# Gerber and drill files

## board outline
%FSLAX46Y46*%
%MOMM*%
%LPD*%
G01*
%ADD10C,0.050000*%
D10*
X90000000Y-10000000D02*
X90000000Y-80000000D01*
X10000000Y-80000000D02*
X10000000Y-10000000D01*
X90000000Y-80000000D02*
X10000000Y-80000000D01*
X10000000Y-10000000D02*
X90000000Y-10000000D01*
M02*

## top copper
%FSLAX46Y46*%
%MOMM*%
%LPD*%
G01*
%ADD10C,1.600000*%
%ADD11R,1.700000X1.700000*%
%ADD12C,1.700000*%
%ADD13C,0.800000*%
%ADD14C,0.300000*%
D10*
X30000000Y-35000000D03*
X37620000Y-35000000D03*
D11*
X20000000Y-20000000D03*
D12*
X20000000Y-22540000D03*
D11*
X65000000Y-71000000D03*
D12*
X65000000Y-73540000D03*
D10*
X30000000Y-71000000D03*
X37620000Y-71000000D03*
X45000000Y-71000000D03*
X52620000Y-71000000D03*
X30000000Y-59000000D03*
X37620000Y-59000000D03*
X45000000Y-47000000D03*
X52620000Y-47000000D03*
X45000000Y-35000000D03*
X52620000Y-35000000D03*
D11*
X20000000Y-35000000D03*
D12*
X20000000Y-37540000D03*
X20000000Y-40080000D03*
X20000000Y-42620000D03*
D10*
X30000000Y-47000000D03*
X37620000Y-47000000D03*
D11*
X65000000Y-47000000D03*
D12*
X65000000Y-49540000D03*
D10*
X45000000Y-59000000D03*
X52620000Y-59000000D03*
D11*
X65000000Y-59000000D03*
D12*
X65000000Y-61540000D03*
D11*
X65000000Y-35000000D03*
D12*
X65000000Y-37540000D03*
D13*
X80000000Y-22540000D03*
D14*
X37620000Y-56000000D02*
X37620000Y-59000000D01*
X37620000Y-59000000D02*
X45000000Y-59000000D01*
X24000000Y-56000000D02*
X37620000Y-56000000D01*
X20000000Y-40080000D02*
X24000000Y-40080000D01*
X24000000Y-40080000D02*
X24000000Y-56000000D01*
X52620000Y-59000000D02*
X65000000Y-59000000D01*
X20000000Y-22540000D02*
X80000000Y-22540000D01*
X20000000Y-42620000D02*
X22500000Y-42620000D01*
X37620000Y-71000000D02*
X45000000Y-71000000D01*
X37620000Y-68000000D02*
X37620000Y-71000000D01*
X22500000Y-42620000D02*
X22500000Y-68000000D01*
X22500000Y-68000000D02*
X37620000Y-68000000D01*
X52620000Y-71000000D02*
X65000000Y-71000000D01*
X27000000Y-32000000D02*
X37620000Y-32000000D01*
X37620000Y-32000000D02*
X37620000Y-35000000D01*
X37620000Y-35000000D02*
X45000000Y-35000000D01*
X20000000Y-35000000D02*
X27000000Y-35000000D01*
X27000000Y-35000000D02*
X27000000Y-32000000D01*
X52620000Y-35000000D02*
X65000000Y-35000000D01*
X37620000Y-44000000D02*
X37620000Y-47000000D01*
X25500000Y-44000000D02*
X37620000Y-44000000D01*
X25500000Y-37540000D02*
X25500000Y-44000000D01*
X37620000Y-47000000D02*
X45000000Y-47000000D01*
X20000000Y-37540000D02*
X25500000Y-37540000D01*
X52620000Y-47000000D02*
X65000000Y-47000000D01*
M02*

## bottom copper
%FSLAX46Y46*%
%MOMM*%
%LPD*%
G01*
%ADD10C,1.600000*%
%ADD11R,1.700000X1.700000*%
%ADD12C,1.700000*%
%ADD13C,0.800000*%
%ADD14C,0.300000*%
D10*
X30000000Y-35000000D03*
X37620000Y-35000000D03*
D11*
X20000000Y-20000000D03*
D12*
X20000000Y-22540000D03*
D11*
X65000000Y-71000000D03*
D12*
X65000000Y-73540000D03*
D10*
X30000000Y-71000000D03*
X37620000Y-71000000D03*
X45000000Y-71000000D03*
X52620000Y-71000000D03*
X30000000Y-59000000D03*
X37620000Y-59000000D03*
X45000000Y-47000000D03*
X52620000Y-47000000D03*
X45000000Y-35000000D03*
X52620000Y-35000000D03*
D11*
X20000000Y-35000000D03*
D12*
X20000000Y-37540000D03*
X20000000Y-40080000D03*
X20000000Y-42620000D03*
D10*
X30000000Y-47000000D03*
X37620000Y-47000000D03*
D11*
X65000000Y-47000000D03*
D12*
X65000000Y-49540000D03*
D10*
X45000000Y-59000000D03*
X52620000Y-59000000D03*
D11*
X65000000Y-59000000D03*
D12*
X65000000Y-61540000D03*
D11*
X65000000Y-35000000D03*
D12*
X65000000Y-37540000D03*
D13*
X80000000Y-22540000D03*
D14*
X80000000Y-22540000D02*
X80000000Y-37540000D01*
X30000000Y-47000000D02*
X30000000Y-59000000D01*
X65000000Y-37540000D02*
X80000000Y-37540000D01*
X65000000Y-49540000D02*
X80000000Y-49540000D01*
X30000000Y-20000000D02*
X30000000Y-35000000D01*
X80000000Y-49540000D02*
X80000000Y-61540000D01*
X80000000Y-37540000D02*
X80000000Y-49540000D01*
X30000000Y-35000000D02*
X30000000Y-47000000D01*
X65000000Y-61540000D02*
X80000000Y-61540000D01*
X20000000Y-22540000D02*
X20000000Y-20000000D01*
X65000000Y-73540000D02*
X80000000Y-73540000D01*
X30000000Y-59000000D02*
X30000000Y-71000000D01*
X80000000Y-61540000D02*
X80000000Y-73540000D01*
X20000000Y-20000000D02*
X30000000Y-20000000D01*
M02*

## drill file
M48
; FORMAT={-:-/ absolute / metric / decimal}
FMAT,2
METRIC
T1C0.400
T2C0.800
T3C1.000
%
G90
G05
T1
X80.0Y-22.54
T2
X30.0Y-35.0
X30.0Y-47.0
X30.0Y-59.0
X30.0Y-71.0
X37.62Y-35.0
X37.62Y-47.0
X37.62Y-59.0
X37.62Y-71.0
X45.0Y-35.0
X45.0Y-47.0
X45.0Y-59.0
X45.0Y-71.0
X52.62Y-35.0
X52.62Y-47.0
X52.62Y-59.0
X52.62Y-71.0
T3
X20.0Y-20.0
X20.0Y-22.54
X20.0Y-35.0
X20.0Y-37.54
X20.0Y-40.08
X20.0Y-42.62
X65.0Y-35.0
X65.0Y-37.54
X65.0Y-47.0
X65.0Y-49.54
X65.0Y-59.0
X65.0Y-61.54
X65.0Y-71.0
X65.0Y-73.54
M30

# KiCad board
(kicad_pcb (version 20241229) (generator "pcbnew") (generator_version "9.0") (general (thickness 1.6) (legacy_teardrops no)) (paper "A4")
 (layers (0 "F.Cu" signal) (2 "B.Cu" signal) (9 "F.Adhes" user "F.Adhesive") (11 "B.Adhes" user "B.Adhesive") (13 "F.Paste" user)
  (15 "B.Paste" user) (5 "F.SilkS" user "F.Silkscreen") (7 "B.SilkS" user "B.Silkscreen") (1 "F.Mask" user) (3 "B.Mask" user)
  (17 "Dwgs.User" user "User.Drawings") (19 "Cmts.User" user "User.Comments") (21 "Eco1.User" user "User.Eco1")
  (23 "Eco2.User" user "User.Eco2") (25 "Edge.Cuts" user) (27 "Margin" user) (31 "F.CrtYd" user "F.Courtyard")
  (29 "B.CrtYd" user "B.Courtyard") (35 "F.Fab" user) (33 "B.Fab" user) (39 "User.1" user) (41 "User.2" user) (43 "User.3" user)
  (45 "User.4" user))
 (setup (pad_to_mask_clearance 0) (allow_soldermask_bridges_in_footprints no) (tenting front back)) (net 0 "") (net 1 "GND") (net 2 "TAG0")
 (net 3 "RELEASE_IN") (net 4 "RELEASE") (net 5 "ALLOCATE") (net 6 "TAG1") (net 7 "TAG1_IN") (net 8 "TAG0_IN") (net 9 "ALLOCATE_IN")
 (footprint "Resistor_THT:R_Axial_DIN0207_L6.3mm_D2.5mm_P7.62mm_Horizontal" (layer "F.Cu") (at 30 35)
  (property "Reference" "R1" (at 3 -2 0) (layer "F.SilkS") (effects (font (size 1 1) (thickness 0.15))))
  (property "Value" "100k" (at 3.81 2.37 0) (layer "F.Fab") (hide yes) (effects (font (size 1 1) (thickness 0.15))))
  (pad "1" thru_hole circle (at 0 0) (size 1.6 1.6) (drill 0.8) (layers "*.Cu" "*.Mask") (remove_unused_layers no) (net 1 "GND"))
  (pad "2" thru_hole circle (at 7.62 0) (size 1.6 1.6) (drill 0.8) (layers "*.Cu" "*.Mask") (remove_unused_layers no) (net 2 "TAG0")))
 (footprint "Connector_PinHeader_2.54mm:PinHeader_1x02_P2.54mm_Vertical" (layer "F.Cu") (at 20 20)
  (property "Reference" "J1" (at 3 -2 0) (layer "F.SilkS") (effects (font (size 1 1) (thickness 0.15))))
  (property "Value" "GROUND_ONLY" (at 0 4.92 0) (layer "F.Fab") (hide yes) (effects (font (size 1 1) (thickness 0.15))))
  (pad "1" thru_hole rect (at 0 0) (size 1.7 1.7) (drill 1) (layers "*.Cu" "*.Mask") (remove_unused_layers no) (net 1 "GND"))
  (pad "2" thru_hole circle (at 0 2.54) (size 1.7 1.7) (drill 1) (layers "*.Cu" "*.Mask") (remove_unused_layers no) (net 1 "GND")))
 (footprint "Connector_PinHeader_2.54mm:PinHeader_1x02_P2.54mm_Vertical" (layer "F.Cu") (at 65 71)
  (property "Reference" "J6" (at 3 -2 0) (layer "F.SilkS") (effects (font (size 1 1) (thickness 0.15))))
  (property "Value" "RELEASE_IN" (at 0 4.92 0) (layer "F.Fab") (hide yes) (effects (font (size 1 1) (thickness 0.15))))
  (pad "1" thru_hole rect (at 0 0) (size 1.7 1.7) (drill 1) (layers "*.Cu" "*.Mask") (remove_unused_layers no) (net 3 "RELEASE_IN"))
  (pad "2" thru_hole circle (at 0 2.54) (size 1.7 1.7) (drill 1) (layers "*.Cu" "*.Mask") (remove_unused_layers no) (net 1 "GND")))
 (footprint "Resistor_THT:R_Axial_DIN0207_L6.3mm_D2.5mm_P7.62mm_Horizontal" (layer "F.Cu") (at 30 71)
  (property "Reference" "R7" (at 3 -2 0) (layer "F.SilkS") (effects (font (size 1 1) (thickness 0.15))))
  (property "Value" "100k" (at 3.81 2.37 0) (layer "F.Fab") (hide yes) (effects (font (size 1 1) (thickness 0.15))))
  (pad "1" thru_hole circle (at 0 0) (size 1.6 1.6) (drill 0.8) (layers "*.Cu" "*.Mask") (remove_unused_layers no) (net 1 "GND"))
  (pad "2" thru_hole circle (at 7.62 0) (size 1.6 1.6) (drill 0.8) (layers "*.Cu" "*.Mask") (remove_unused_layers no) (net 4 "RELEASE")))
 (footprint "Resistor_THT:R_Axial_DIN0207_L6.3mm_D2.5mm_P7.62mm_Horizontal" (layer "F.Cu") (at 45 71)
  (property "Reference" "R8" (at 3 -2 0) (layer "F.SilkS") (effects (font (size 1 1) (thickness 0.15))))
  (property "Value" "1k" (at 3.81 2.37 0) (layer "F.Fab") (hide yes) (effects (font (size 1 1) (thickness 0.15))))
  (pad "1" thru_hole circle (at 0 0) (size 1.6 1.6) (drill 0.8) (layers "*.Cu" "*.Mask") (remove_unused_layers no) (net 4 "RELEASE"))
  (pad "2" thru_hole circle (at 7.62 0) (size 1.6 1.6) (drill 0.8) (layers "*.Cu" "*.Mask") (remove_unused_layers no) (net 3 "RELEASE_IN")))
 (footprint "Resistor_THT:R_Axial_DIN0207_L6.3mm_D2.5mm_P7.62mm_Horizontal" (layer "F.Cu") (at 30 59)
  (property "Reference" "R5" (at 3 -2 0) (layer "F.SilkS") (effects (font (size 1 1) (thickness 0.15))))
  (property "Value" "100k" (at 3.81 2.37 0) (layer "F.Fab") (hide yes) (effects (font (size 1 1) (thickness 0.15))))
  (pad "1" thru_hole circle (at 0 0) (size 1.6 1.6) (drill 0.8) (layers "*.Cu" "*.Mask") (remove_unused_layers no) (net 1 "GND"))
  (pad "2" thru_hole circle (at 7.62 0) (size 1.6 1.6) (drill 0.8) (layers "*.Cu" "*.Mask") (remove_unused_layers no) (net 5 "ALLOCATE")))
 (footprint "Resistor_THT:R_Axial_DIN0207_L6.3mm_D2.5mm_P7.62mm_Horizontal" (layer "F.Cu") (at 45 47)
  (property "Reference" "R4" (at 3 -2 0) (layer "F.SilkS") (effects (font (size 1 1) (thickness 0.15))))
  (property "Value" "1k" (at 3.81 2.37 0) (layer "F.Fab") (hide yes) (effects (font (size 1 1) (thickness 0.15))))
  (pad "1" thru_hole circle (at 0 0) (size 1.6 1.6) (drill 0.8) (layers "*.Cu" "*.Mask") (remove_unused_layers no) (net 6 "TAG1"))
  (pad "2" thru_hole circle (at 7.62 0) (size 1.6 1.6) (drill 0.8) (layers "*.Cu" "*.Mask") (remove_unused_layers no) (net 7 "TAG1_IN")))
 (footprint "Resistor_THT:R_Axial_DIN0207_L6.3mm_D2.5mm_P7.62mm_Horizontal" (layer "F.Cu") (at 45 35)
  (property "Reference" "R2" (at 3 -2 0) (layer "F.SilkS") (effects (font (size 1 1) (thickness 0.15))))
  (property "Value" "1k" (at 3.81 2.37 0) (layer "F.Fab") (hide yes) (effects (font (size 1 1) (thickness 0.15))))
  (pad "1" thru_hole circle (at 0 0) (size 1.6 1.6) (drill 0.8) (layers "*.Cu" "*.Mask") (remove_unused_layers no) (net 2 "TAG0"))
  (pad "2" thru_hole circle (at 7.62 0) (size 1.6 1.6) (drill 0.8) (layers "*.Cu" "*.Mask") (remove_unused_layers no) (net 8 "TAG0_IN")))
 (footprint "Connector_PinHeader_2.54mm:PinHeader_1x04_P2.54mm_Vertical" (layer "F.Cu") (at 20 35)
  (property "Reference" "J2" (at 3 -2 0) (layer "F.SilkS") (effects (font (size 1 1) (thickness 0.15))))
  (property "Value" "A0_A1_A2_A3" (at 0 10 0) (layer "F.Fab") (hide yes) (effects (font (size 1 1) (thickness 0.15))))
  (pad "1" thru_hole rect (at 0 0) (size 1.7 1.7) (drill 1) (layers "*.Cu" "*.Mask") (remove_unused_layers no) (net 2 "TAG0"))
  (pad "2" thru_hole circle (at 0 2.54) (size 1.7 1.7) (drill 1) (layers "*.Cu" "*.Mask") (remove_unused_layers no) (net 6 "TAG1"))
  (pad "3" thru_hole circle (at 0 5.08) (size 1.7 1.7) (drill 1) (layers "*.Cu" "*.Mask") (remove_unused_layers no) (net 5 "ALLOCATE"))
  (pad "4" thru_hole circle (at 0 7.62) (size 1.7 1.7) (drill 1) (layers "*.Cu" "*.Mask") (remove_unused_layers no) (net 4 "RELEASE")))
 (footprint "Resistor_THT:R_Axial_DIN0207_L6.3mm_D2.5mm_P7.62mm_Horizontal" (layer "F.Cu") (at 30 47)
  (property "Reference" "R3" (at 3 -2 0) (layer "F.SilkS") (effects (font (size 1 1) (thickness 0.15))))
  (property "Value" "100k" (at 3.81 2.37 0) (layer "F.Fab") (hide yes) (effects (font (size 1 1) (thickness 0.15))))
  (pad "1" thru_hole circle (at 0 0) (size 1.6 1.6) (drill 0.8) (layers "*.Cu" "*.Mask") (remove_unused_layers no) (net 1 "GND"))
  (pad "2" thru_hole circle (at 7.62 0) (size 1.6 1.6) (drill 0.8) (layers "*.Cu" "*.Mask") (remove_unused_layers no) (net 6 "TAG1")))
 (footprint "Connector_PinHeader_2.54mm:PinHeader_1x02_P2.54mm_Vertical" (layer "F.Cu") (at 65 47)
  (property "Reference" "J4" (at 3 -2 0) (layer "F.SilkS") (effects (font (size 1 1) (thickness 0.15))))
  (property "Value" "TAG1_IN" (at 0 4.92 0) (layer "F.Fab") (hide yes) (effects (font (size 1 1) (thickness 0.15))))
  (pad "1" thru_hole rect (at 0 0) (size 1.7 1.7) (drill 1) (layers "*.Cu" "*.Mask") (remove_unused_layers no) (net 7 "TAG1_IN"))
  (pad "2" thru_hole circle (at 0 2.54) (size 1.7 1.7) (drill 1) (layers "*.Cu" "*.Mask") (remove_unused_layers no) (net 1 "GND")))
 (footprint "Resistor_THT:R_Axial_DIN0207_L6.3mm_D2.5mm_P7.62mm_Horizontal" (layer "F.Cu") (at 45 59)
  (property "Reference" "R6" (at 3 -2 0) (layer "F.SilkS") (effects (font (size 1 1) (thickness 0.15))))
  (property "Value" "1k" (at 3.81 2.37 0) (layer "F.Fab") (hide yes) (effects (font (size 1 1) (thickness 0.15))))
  (pad "1" thru_hole circle (at 0 0) (size 1.6 1.6) (drill 0.8) (layers "*.Cu" "*.Mask") (remove_unused_layers no) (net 5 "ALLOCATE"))
  (pad "2" thru_hole circle (at 7.62 0) (size 1.6 1.6) (drill 0.8) (layers "*.Cu" "*.Mask") (remove_unused_layers no) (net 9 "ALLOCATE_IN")))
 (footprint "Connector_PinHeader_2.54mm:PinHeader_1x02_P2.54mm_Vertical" (layer "F.Cu") (at 65 59)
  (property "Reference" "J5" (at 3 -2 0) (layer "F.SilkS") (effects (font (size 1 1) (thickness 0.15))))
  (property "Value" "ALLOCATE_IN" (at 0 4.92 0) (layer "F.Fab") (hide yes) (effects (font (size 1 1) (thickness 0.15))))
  (pad "1" thru_hole rect (at 0 0) (size 1.7 1.7) (drill 1) (layers "*.Cu" "*.Mask") (remove_unused_layers no) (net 9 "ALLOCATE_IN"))
  (pad "2" thru_hole circle (at 0 2.54) (size 1.7 1.7) (drill 1) (layers "*.Cu" "*.Mask") (remove_unused_layers no) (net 1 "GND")))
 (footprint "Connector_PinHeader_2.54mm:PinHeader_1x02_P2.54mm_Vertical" (layer "F.Cu") (at 65 35)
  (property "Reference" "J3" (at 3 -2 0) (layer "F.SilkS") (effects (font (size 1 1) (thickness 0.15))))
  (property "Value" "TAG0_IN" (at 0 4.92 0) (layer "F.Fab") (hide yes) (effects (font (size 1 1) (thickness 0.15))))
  (pad "1" thru_hole rect (at 0 0) (size 1.7 1.7) (drill 1) (layers "*.Cu" "*.Mask") (remove_unused_layers no) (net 8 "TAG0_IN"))
  (pad "2" thru_hole circle (at 0 2.54) (size 1.7 1.7) (drill 1) (layers "*.Cu" "*.Mask") (remove_unused_layers no) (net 1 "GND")))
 (gr_line (start 90 10) (end 90 80) (stroke (width 0.05) (type default)) (layer "Edge.Cuts"))
 (gr_line (start 10 80) (end 10 10) (stroke (width 0.05) (type default)) (layer "Edge.Cuts"))
 (gr_line (start 90 80) (end 10 80) (stroke (width 0.05) (type default)) (layer "Edge.Cuts"))
 (gr_line (start 10 10) (end 90 10) (stroke (width 0.05) (type default)) (layer "Edge.Cuts"))
 (segment (start 37.62 56) (end 37.62 59) (width 0.3) (layer "F.Cu") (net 5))
 (segment (start 37.62 59) (end 45 59) (width 0.3) (layer "F.Cu") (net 5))
 (segment (start 24 56) (end 37.62 56) (width 0.3) (layer "F.Cu") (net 5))
 (segment (start 20 40.08) (end 24 40.08) (width 0.3) (layer "F.Cu") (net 5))
 (segment (start 24 40.08) (end 24 56) (width 0.3) (layer "F.Cu") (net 5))
 (segment (start 52.62 59) (end 65 59) (width 0.3) (layer "F.Cu") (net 9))
 (segment (start 20 22.54) (end 80 22.54) (width 0.3) (layer "F.Cu") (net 1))
 (via (at 80 22.54) (size 0.8) (drill 0.4) (layers "F.Cu" "B.Cu") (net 1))
 (segment (start 80 22.54) (end 80 37.54) (width 0.3) (layer "B.Cu") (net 1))
 (segment (start 30 47) (end 30 59) (width 0.3) (layer "B.Cu") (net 1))
 (segment (start 65 37.54) (end 80 37.54) (width 0.3) (layer "B.Cu") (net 1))
 (segment (start 65 49.54) (end 80 49.54) (width 0.3) (layer "B.Cu") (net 1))
 (segment (start 30 20) (end 30 35) (width 0.3) (layer "B.Cu") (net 1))
 (segment (start 80 49.54) (end 80 61.54) (width 0.3) (layer "B.Cu") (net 1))
 (segment (start 80 37.54) (end 80 49.54) (width 0.3) (layer "B.Cu") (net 1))
 (segment (start 30 35) (end 30 47) (width 0.3) (layer "B.Cu") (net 1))
 (segment (start 65 61.54) (end 80 61.54) (width 0.3) (layer "B.Cu") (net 1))
 (segment (start 20 22.54) (end 20 20) (width 0.3) (layer "B.Cu") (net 1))
 (segment (start 65 73.54) (end 80 73.54) (width 0.3) (layer "B.Cu") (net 1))
 (segment (start 30 59) (end 30 71) (width 0.3) (layer "B.Cu") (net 1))
 (segment (start 80 61.54) (end 80 73.54) (width 0.3) (layer "B.Cu") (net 1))
 (segment (start 20 20) (end 30 20) (width 0.3) (layer "B.Cu") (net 1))
 (segment (start 20 42.62) (end 22.5 42.62) (width 0.3) (layer "F.Cu") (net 4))
 (segment (start 37.62 71) (end 45 71) (width 0.3) (layer "F.Cu") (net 4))
 (segment (start 37.62 68) (end 37.62 71) (width 0.3) (layer "F.Cu") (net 4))
 (segment (start 22.5 42.62) (end 22.5 68) (width 0.3) (layer "F.Cu") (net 4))
 (segment (start 22.5 68) (end 37.62 68) (width 0.3) (layer "F.Cu") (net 4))
 (segment (start 52.62 71) (end 65 71) (width 0.3) (layer "F.Cu") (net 3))
 (segment (start 27 32) (end 37.62 32) (width 0.3) (layer "F.Cu") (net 2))
 (segment (start 37.62 32) (end 37.62 35) (width 0.3) (layer "F.Cu") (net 2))
 (segment (start 37.62 35) (end 45 35) (width 0.3) (layer "F.Cu") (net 2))
 (segment (start 20 35) (end 27 35) (width 0.3) (layer "F.Cu") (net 2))
 (segment (start 27 35) (end 27 32) (width 0.3) (layer "F.Cu") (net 2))
 (segment (start 52.62 35) (end 65 35) (width 0.3) (layer "F.Cu") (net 8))
 (segment (start 37.62 44) (end 37.62 47) (width 0.3) (layer "F.Cu") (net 6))
 (segment (start 25.5 44) (end 37.62 44) (width 0.3) (layer "F.Cu") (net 6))
 (segment (start 25.5 37.54) (end 25.5 44) (width 0.3) (layer "F.Cu") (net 6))
 (segment (start 37.62 47) (end 45 47) (width 0.3) (layer "F.Cu") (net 6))
 (segment (start 20 37.54) (end 25.5 37.54) (width 0.3) (layer "F.Cu") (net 6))
 (segment (start 52.62 47) (end 65 47) (width 0.3) (layer "F.Cu") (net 7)))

